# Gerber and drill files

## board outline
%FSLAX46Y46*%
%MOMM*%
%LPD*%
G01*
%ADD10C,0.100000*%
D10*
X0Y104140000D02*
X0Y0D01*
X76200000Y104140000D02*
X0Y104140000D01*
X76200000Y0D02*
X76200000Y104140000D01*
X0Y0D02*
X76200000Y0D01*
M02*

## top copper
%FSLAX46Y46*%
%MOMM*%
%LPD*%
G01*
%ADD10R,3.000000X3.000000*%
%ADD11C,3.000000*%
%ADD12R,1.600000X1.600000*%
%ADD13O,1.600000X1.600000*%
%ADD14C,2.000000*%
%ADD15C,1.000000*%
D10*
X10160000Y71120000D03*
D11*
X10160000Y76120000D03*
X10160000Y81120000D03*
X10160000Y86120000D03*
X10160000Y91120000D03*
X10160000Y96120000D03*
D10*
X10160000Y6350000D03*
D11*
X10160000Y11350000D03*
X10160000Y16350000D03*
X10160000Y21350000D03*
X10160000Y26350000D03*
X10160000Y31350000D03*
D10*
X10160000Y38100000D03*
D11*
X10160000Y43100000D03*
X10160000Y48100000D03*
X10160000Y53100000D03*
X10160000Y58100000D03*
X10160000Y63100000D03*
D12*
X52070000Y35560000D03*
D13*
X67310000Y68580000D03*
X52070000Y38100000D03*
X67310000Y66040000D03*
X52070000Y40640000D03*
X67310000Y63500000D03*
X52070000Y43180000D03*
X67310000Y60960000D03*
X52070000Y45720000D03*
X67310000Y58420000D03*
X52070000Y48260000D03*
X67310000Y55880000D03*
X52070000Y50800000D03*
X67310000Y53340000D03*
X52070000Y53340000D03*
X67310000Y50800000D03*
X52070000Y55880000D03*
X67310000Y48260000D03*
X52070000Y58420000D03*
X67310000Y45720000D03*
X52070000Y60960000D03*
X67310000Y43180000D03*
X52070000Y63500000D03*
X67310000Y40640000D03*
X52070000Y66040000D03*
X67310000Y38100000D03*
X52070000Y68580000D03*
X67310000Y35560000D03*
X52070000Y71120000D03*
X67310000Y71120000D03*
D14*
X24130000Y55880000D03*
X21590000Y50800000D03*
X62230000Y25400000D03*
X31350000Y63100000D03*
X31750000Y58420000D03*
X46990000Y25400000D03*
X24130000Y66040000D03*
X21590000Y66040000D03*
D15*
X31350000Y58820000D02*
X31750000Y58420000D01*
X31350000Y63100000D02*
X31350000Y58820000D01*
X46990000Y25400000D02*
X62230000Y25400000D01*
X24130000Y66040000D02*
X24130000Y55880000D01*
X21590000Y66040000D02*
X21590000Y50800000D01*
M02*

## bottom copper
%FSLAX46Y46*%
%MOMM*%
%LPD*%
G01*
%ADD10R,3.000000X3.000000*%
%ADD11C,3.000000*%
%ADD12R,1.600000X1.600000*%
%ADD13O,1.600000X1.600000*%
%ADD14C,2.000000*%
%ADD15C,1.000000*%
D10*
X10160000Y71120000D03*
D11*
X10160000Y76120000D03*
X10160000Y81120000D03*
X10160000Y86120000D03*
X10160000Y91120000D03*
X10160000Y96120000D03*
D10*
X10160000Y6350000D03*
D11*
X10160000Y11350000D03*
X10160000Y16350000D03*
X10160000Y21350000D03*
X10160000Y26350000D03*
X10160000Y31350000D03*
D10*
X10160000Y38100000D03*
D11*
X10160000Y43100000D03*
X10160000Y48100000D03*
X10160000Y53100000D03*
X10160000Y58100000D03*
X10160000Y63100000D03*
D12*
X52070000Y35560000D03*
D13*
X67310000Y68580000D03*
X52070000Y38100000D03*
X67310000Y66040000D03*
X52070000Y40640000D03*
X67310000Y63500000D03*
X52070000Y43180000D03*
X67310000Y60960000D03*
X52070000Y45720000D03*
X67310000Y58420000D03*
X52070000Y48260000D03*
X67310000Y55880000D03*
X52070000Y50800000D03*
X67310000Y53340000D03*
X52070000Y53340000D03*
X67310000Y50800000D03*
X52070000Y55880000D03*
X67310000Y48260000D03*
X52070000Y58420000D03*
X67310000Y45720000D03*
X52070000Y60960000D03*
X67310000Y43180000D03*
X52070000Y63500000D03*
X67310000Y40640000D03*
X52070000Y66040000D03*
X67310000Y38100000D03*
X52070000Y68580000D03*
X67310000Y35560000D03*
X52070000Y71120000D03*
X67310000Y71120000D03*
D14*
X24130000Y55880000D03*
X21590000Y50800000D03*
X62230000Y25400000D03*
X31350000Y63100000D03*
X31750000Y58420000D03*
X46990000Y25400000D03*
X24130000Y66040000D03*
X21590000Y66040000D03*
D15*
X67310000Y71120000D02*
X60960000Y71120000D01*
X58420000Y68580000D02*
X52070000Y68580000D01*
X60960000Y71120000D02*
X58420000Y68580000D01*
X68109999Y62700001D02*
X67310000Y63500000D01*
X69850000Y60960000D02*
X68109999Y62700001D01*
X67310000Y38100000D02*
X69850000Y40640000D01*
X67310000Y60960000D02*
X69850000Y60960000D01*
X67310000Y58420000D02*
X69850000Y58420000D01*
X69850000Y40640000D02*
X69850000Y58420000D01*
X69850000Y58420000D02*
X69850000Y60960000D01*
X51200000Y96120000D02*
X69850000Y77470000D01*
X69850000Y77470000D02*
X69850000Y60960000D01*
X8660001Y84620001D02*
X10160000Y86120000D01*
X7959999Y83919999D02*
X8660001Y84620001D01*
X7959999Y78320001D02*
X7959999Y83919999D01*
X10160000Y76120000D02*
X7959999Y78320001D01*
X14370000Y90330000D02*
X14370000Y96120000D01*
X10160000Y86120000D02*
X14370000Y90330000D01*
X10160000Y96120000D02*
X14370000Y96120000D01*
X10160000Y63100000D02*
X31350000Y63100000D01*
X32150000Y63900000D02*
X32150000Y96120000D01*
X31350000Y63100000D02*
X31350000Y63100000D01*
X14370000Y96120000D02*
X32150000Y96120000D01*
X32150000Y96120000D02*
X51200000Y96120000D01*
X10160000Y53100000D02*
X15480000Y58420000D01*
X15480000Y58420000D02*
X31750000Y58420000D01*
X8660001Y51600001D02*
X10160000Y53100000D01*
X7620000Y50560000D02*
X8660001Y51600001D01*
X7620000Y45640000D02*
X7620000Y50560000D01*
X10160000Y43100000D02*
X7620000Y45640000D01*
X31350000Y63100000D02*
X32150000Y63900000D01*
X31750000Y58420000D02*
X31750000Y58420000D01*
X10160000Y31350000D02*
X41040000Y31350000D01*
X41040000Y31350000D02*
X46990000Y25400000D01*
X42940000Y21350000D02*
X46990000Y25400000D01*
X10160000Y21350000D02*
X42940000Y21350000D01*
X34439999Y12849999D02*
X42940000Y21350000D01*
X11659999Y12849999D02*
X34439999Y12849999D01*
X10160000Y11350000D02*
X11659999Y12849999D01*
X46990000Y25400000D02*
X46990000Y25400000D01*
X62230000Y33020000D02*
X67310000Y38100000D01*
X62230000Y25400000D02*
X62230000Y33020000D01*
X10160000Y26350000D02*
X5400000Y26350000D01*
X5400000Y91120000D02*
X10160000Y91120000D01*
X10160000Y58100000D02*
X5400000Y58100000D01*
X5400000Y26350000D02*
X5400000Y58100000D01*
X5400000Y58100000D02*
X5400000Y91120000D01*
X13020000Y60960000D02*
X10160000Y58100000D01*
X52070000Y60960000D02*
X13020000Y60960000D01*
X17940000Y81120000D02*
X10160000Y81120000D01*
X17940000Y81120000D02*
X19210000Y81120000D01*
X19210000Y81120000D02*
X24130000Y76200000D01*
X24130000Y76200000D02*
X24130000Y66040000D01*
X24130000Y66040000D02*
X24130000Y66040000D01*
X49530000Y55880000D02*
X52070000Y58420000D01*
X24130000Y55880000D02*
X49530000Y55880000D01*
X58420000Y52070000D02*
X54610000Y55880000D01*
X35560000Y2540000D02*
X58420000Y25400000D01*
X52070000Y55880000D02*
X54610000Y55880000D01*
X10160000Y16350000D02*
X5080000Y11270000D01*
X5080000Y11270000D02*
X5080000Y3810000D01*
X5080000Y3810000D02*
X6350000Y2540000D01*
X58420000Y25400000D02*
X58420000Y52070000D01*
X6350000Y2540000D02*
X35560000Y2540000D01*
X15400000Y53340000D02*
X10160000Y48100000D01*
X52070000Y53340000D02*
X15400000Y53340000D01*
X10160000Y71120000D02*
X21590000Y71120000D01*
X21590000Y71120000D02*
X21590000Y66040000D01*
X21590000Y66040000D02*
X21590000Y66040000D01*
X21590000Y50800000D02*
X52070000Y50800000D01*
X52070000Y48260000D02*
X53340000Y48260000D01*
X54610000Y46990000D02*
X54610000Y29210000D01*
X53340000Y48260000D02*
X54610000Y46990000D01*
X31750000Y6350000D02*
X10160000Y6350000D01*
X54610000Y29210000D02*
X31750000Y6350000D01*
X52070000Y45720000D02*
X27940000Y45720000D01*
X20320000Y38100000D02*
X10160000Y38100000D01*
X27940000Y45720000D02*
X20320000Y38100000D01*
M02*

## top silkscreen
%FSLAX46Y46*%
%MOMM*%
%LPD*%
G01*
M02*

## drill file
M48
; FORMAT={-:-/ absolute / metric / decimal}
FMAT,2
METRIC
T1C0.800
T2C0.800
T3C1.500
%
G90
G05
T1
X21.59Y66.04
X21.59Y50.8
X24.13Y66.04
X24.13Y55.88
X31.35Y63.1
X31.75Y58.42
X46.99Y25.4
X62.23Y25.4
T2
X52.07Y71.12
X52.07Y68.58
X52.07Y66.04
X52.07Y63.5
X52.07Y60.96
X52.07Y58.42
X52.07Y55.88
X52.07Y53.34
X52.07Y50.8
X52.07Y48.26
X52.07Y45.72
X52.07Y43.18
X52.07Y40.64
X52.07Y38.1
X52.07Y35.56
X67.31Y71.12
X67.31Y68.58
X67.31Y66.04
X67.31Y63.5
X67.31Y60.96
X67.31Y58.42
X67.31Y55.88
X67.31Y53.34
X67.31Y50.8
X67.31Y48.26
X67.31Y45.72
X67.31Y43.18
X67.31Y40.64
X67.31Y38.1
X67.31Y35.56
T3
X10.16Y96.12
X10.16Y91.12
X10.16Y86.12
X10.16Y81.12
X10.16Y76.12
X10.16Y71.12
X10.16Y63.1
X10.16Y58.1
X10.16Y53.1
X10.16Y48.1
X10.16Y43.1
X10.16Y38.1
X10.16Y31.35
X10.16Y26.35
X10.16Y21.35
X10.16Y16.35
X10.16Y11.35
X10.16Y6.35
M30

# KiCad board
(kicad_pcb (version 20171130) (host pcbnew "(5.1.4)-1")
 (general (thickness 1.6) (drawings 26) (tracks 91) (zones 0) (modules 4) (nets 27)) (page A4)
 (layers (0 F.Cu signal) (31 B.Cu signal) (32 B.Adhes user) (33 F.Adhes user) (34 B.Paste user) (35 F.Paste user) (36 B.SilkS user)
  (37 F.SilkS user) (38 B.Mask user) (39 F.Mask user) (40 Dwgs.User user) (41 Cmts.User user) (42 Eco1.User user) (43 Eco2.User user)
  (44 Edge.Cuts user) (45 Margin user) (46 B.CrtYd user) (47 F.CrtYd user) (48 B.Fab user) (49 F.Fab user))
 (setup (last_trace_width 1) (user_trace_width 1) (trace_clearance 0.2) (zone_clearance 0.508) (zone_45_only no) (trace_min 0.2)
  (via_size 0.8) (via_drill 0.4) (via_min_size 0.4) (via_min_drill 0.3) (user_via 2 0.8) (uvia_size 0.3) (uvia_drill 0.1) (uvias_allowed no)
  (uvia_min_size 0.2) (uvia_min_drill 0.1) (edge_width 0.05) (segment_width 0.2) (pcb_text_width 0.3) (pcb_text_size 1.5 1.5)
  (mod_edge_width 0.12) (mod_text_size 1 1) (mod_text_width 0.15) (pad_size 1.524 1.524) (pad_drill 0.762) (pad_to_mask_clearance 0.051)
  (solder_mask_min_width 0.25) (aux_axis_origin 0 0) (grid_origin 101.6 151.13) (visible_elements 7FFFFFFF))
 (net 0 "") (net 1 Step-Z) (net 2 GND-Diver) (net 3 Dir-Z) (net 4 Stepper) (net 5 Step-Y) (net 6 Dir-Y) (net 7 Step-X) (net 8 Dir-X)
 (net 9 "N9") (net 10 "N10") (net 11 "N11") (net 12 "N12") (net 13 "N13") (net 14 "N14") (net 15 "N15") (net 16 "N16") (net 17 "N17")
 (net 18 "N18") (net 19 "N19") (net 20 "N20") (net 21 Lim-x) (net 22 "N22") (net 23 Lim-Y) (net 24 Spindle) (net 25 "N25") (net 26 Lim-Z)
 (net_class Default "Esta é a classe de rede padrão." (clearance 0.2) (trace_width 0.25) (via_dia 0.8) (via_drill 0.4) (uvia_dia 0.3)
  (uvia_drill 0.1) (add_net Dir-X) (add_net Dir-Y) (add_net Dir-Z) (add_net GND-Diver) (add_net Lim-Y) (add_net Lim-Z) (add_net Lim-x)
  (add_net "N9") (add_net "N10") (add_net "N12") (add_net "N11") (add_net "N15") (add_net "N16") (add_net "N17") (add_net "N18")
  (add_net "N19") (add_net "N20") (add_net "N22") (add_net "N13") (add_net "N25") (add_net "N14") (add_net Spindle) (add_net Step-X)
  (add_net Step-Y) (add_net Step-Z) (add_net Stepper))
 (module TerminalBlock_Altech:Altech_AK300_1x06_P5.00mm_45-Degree (layer B.Cu) (at 10.16 -71.12 90)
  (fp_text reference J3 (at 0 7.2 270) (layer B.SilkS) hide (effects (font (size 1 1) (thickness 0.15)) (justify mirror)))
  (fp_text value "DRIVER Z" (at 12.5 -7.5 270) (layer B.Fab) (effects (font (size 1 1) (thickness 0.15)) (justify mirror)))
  (pad 1 thru_hole rect (at 0 0 90) (size 3 3) (drill 1.5) (layers *.Cu *.Mask) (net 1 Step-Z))
  (pad 2 thru_hole circle (at 5 0 90) (size 3 3) (drill 1.5) (layers *.Cu *.Mask) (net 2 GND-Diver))
  (pad 3 thru_hole circle (at 10 0 90) (size 3 3) (drill 1.5) (layers *.Cu *.Mask) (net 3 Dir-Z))
  (pad 4 thru_hole circle (at 15 0 90) (size 3 3) (drill 1.5) (layers *.Cu *.Mask) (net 2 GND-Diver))
  (pad 5 thru_hole circle (at 20 0 90) (size 3 3) (drill 1.5) (layers *.Cu *.Mask) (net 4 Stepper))
  (pad 6 thru_hole circle (at 25 0 90) (size 3 3) (drill 1.5) (layers *.Cu *.Mask) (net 2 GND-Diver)))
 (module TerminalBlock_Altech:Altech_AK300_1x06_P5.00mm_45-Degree (layer B.Cu) (at 10.16 -6.35 90)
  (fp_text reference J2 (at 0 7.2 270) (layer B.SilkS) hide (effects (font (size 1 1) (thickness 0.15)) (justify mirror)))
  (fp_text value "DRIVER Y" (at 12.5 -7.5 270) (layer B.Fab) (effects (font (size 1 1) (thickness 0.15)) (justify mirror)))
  (pad 1 thru_hole rect (at 0 0 90) (size 3 3) (drill 1.5) (layers *.Cu *.Mask) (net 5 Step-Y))
  (pad 2 thru_hole circle (at 5 0 90) (size 3 3) (drill 1.5) (layers *.Cu *.Mask) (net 2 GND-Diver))
  (pad 3 thru_hole circle (at 10 0 90) (size 3 3) (drill 1.5) (layers *.Cu *.Mask) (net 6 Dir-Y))
  (pad 4 thru_hole circle (at 15 0 90) (size 3 3) (drill 1.5) (layers *.Cu *.Mask) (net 2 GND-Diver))
  (pad 5 thru_hole circle (at 20 0 90) (size 3 3) (drill 1.5) (layers *.Cu *.Mask) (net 4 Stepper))
  (pad 6 thru_hole circle (at 25 0 90) (size 3 3) (drill 1.5) (layers *.Cu *.Mask) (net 2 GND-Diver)))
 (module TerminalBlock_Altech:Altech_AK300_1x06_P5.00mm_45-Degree (layer B.Cu) (at 10.16 -38.1 90)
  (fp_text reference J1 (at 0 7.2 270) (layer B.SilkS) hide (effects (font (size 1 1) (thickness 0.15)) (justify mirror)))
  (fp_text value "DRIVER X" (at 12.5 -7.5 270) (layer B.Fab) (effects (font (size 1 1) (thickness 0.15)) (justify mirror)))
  (pad 1 thru_hole rect (at 0 0 90) (size 3 3) (drill 1.5) (layers *.Cu *.Mask) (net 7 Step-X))
  (pad 2 thru_hole circle (at 5 0 90) (size 3 3) (drill 1.5) (layers *.Cu *.Mask) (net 2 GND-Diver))
  (pad 3 thru_hole circle (at 10 0 90) (size 3 3) (drill 1.5) (layers *.Cu *.Mask) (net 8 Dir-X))
  (pad 4 thru_hole circle (at 15 0 90) (size 3 3) (drill 1.5) (layers *.Cu *.Mask) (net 2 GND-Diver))
  (pad 5 thru_hole circle (at 20 0 90) (size 3 3) (drill 1.5) (layers *.Cu *.Mask) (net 4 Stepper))
  (pad 6 thru_hole circle (at 25 0 90) (size 3 3) (drill 1.5) (layers *.Cu *.Mask) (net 2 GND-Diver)))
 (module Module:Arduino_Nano (layer B.Cu) (at 52.07 -35.56)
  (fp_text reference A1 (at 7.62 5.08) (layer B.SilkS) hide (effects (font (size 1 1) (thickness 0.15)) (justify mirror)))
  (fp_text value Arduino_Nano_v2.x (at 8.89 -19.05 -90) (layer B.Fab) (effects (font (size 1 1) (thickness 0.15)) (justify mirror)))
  (pad 1 thru_hole rect (at 0 0) (size 1.6 1.6) (drill 0.8) (layers *.Cu *.Mask) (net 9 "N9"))
  (pad 17 thru_hole oval (at 15.24 -33.02) (size 1.6 1.6) (drill 0.8) (layers *.Cu *.Mask) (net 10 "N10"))
  (pad 2 thru_hole oval (at 0 -2.54) (size 1.6 1.6) (drill 0.8) (layers *.Cu *.Mask) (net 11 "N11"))
  (pad 18 thru_hole oval (at 15.24 -30.48) (size 1.6 1.6) (drill 0.8) (layers *.Cu *.Mask) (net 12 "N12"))
  (pad 3 thru_hole oval (at 0 -5.08) (size 1.6 1.6) (drill 0.8) (layers *.Cu *.Mask) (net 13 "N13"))
  (pad 19 thru_hole oval (at 15.24 -27.94) (size 1.6 1.6) (drill 0.8) (layers *.Cu *.Mask) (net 2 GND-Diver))
  (pad 4 thru_hole oval (at 0 -7.62) (size 1.6 1.6) (drill 0.8) (layers *.Cu *.Mask) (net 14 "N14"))
  (pad 20 thru_hole oval (at 15.24 -25.4) (size 1.6 1.6) (drill 0.8) (layers *.Cu *.Mask) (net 2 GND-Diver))
  (pad 5 thru_hole oval (at 0 -10.16) (size 1.6 1.6) (drill 0.8) (layers *.Cu *.Mask) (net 7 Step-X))
  (pad 21 thru_hole oval (at 15.24 -22.86) (size 1.6 1.6) (drill 0.8) (layers *.Cu *.Mask) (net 2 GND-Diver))
  (pad 6 thru_hole oval (at 0 -12.7) (size 1.6 1.6) (drill 0.8) (layers *.Cu *.Mask) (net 5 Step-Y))
  (pad 22 thru_hole oval (at 15.24 -20.32) (size 1.6 1.6) (drill 0.8) (layers *.Cu *.Mask) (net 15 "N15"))
  (pad 7 thru_hole oval (at 0 -15.24) (size 1.6 1.6) (drill 0.8) (layers *.Cu *.Mask) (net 1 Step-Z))
  (pad 23 thru_hole oval (at 15.24 -17.78) (size 1.6 1.6) (drill 0.8) (layers *.Cu *.Mask) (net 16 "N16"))
  (pad 8 thru_hole oval (at 0 -17.78) (size 1.6 1.6) (drill 0.8) (layers *.Cu *.Mask) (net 8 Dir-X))
  (pad 24 thru_hole oval (at 15.24 -15.24) (size 1.6 1.6) (drill 0.8) (layers *.Cu *.Mask) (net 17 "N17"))
  (pad 9 thru_hole oval (at 0 -20.32) (size 1.6 1.6) (drill 0.8) (layers *.Cu *.Mask) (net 6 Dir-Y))
  (pad 25 thru_hole oval (at 15.24 -12.7) (size 1.6 1.6) (drill 0.8) (layers *.Cu *.Mask) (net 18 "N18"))
  (pad 10 thru_hole oval (at 0 -22.86) (size 1.6 1.6) (drill 0.8) (layers *.Cu *.Mask) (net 3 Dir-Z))
  (pad 26 thru_hole oval (at 15.24 -10.16) (size 1.6 1.6) (drill 0.8) (layers *.Cu *.Mask) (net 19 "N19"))
  (pad 11 thru_hole oval (at 0 -25.4) (size 1.6 1.6) (drill 0.8) (layers *.Cu *.Mask) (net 4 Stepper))
  (pad 27 thru_hole oval (at 15.24 -7.62) (size 1.6 1.6) (drill 0.8) (layers *.Cu *.Mask) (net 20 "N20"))
  (pad 12 thru_hole oval (at 0 -27.94) (size 1.6 1.6) (drill 0.8) (layers *.Cu *.Mask) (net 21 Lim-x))
  (pad 28 thru_hole oval (at 15.24 -5.08) (size 1.6 1.6) (drill 0.8) (layers *.Cu *.Mask) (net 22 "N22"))
  (pad 13 thru_hole oval (at 0 -30.48) (size 1.6 1.6) (drill 0.8) (layers *.Cu *.Mask) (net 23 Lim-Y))
  (pad 29 thru_hole oval (at 15.24 -2.54) (size 1.6 1.6) (drill 0.8) (layers *.Cu *.Mask) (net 2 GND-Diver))
  (pad 14 thru_hole oval (at 0 -33.02) (size 1.6 1.6) (drill 0.8) (layers *.Cu *.Mask) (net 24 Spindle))
  (pad 30 thru_hole oval (at 15.24 0) (size 1.6 1.6) (drill 0.8) (layers *.Cu *.Mask) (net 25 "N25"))
  (pad 15 thru_hole oval (at 0 -35.56) (size 1.6 1.6) (drill 0.8) (layers *.Cu *.Mask) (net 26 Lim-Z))
  (pad 16 thru_hole oval (at 15.24 -35.56) (size 1.6 1.6) (drill 0.8) (layers *.Cu *.Mask) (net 24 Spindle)))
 (gr_line (start 0 -104.14) (end 0 0) (layer Edge.Cuts) (width 0.1))
 (gr_line (start 76.2 -104.14) (end 0 -104.14) (layer Edge.Cuts) (width 0.1))
 (gr_line (start 76.2 0) (end 76.2 -104.14) (layer Edge.Cuts) (width 0.1))
 (gr_line (start 0 0) (end 76.2 0) (layer Edge.Cuts) (width 0.1))
 (via (at 24.13 -55.88) (size 2) (drill 0.8) (layers F.Cu B.Cu) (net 3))
 (via (at 21.59 -50.8) (size 2) (drill 0.8) (layers F.Cu B.Cu) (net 1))
 (via (at 62.23 -25.4) (size 2) (drill 0.8) (layers F.Cu B.Cu) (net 2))
 (segment (start 67.31 -71.12) (end 60.96 -71.12) (width 1) (layer B.Cu) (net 24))
 (segment (start 58.42 -68.58) (end 52.07 -68.58) (width 1) (layer B.Cu) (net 24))
 (segment (start 60.96 -71.12) (end 58.42 -68.58) (width 1) (layer B.Cu) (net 24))
 (segment (start 68.109999 -62.700001) (end 67.31 -63.5) (width 1) (layer B.Cu) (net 2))
 (segment (start 69.85 -60.96) (end 68.109999 -62.700001) (width 1) (layer B.Cu) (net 2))
 (segment (start 67.31 -38.1) (end 69.85 -40.64) (width 1) (layer B.Cu) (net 2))
 (segment (start 67.31 -60.96) (end 69.85 -60.96) (width 1) (layer B.Cu) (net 2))
 (segment (start 67.31 -58.42) (end 69.85 -58.42) (width 1) (layer B.Cu) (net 2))
 (segment (start 69.85 -40.64) (end 69.85 -58.42) (width 1) (layer B.Cu) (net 2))
 (segment (start 69.85 -58.42) (end 69.85 -60.96) (width 1) (layer B.Cu) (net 2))
 (segment (start 51.2 -96.12) (end 69.85 -77.47) (width 1) (layer B.Cu) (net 2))
 (segment (start 69.85 -77.47) (end 69.85 -60.96) (width 1) (layer B.Cu) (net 2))
 (segment (start 8.660001 -84.620001) (end 10.16 -86.12) (width 1) (layer B.Cu) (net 2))
 (segment (start 7.959999 -83.919999) (end 8.660001 -84.620001) (width 1) (layer B.Cu) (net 2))
 (segment (start 7.959999 -78.320001) (end 7.959999 -83.919999) (width 1) (layer B.Cu) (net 2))
 (segment (start 10.16 -76.12) (end 7.959999 -78.320001) (width 1) (layer B.Cu) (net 2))
 (segment (start 14.37 -90.33) (end 14.37 -96.12) (width 1) (layer B.Cu) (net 2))
 (segment (start 10.16 -86.12) (end 14.37 -90.33) (width 1) (layer B.Cu) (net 2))
 (segment (start 10.16 -96.12) (end 14.37 -96.12) (width 1) (layer B.Cu) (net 2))
 (segment (start 10.16 -63.1) (end 31.35 -63.1) (width 1) (layer B.Cu) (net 2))
 (segment (start 32.15 -63.9) (end 32.15 -96.12) (width 1) (layer B.Cu) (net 2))
 (segment (start 31.35 -63.1) (end 31.35 -63.1) (width 1) (layer B.Cu) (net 2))
 (segment (start 14.37 -96.12) (end 32.15 -96.12) (width 1) (layer B.Cu) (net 2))
 (segment (start 32.15 -96.12) (end 51.2 -96.12) (width 1) (layer B.Cu) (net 2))
 (segment (start 10.16 -53.1) (end 15.48 -58.42) (width 1) (layer B.Cu) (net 2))
 (segment (start 15.48 -58.42) (end 31.75 -58.42) (width 1) (layer B.Cu) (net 2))
 (segment (start 8.660001 -51.600001) (end 10.16 -53.1) (width 1) (layer B.Cu) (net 2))
 (segment (start 7.62 -50.56) (end 8.660001 -51.600001) (width 1) (layer B.Cu) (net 2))
 (segment (start 7.62 -45.64) (end 7.62 -50.56) (width 1) (layer B.Cu) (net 2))
 (segment (start 10.16 -43.1) (end 7.62 -45.64) (width 1) (layer B.Cu) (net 2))
 (segment (start 31.35 -63.1) (end 32.15 -63.9) (width 1) (layer B.Cu) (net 2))
 (via (at 31.35 -63.1) (size 2) (drill 0.8) (layers F.Cu B.Cu) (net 2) (status 1000000))
 (segment (start 31.75 -58.42) (end 31.75 -58.42) (width 1) (layer B.Cu) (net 2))
 (via (at 31.75 -58.42) (size 2) (drill 0.8) (layers F.Cu B.Cu) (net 2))
 (segment (start 10.16 -31.35) (end 41.04 -31.35) (width 1) (layer B.Cu) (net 2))
 (segment (start 41.04 -31.35) (end 46.99 -25.4) (width 1) (layer B.Cu) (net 2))
 (segment (start 42.94 -21.35) (end 46.99 -25.4) (width 1) (layer B.Cu) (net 2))
 (segment (start 10.16 -21.35) (end 42.94 -21.35) (width 1) (layer B.Cu) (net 2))
 (segment (start 34.439999 -12.849999) (end 42.94 -21.35) (width 1) (layer B.Cu) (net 2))
 (segment (start 11.659999 -12.849999) (end 34.439999 -12.849999) (width 1) (layer B.Cu) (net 2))
 (segment (start 10.16 -11.35) (end 11.659999 -12.849999) (width 1) (layer B.Cu) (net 2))
 (segment (start 46.99 -25.4) (end 46.99 -25.4) (width 1) (layer B.Cu) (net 2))
 (via (at 46.99 -25.4) (size 2) (drill 0.8) (layers F.Cu B.Cu) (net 2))
 (segment (start 62.23 -33.02) (end 67.31 -38.1) (width 1) (layer B.Cu) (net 2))
 (segment (start 62.23 -25.4) (end 62.23 -33.02) (width 1) (layer B.Cu) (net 2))
 (segment (start 31.35 -58.82) (end 31.75 -58.42) (width 1) (layer F.Cu) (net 2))
 (segment (start 31.35 -63.1) (end 31.35 -58.82) (width 1) (layer F.Cu) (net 2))
 (segment (start 46.99 -25.4) (end 62.23 -25.4) (width 1) (layer F.Cu) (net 2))
 (segment (start 10.16 -26.35) (end 5.4 -26.35) (width 1) (layer B.Cu) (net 4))
 (segment (start 5.4 -91.12) (end 10.16 -91.12) (width 1) (layer B.Cu) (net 4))
 (segment (start 10.16 -58.1) (end 5.4 -58.1) (width 1) (layer B.Cu) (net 4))
 (segment (start 5.4 -26.35) (end 5.4 -58.1) (width 1) (layer B.Cu) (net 4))
 (segment (start 5.4 -58.1) (end 5.4 -91.12) (width 1) (layer B.Cu) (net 4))
 (segment (start 13.02 -60.96) (end 10.16 -58.1) (width 1) (layer B.Cu) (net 4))
 (segment (start 52.07 -60.96) (end 13.02 -60.96) (width 1) (layer B.Cu) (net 4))
 (segment (start 17.94 -81.12) (end 10.16 -81.12) (width 1) (layer B.Cu) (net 3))
 (segment (start 17.94 -81.12) (end 19.21 -81.12) (width 1) (layer B.Cu) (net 3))
 (segment (start 19.21 -81.12) (end 24.13 -76.2) (width 1) (layer B.Cu) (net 3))
 (segment (start 24.13 -76.2) (end 24.13 -66.04) (width 1) (layer B.Cu) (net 3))
 (segment (start 24.13 -66.04) (end 24.13 -66.04) (width 1) (layer B.Cu) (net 3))
 (via (at 24.13 -66.04) (size 2) (drill 0.8) (layers F.Cu B.Cu) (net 3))
 (segment (start 49.53 -55.88) (end 52.07 -58.42) (width 1) (layer B.Cu) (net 3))
 (segment (start 24.13 -55.88) (end 49.53 -55.88) (width 1) (layer B.Cu) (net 3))
 (segment (start 24.13 -66.04) (end 24.13 -55.88) (width 1) (layer F.Cu) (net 3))
 (segment (start 58.42 -52.07) (end 54.61 -55.88) (width 1) (layer B.Cu) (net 6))
 (segment (start 35.56 -2.54) (end 58.42 -25.4) (width 1) (layer B.Cu) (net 6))
 (segment (start 52.07 -55.88) (end 54.61 -55.88) (width 1) (layer B.Cu) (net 6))
 (segment (start 10.16 -16.35) (end 5.08 -11.27) (width 1) (layer B.Cu) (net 6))
 (segment (start 5.08 -11.27) (end 5.08 -3.81) (width 1) (layer B.Cu) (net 6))
 (segment (start 5.08 -3.81) (end 6.35 -2.54) (width 1) (layer B.Cu) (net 6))
 (segment (start 58.42 -25.4) (end 58.42 -52.07) (width 1) (layer B.Cu) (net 6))
 (segment (start 6.35 -2.54) (end 35.56 -2.54) (width 1) (layer B.Cu) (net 6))
 (segment (start 15.4 -53.34) (end 10.16 -48.1) (width 1) (layer B.Cu) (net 8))
 (segment (start 52.07 -53.34) (end 15.4 -53.34) (width 1) (layer B.Cu) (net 8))
 (segment (start 10.16 -71.12) (end 21.59 -71.12) (width 1) (layer B.Cu) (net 1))
 (segment (start 21.59 -71.12) (end 21.59 -66.04) (width 1) (layer B.Cu) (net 1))
 (segment (start 21.59 -66.04) (end 21.59 -66.04) (width 1) (layer B.Cu) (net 1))
 (via (at 21.59 -66.04) (size 2) (drill 0.8) (layers F.Cu B.Cu) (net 1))
 (segment (start 21.59 -50.8) (end 52.07 -50.8) (width 1) (layer B.Cu) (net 1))
 (segment (start 21.59 -66.04) (end 21.59 -50.8) (width 1) (layer F.Cu) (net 1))
 (segment (start 52.07 -48.26) (end 53.34 -48.26) (width 1) (layer B.Cu) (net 5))
 (segment (start 54.61 -46.99) (end 54.61 -29.21) (width 1) (layer B.Cu) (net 5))
 (segment (start 53.34 -48.26) (end 54.61 -46.99) (width 1) (layer B.Cu) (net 5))
 (segment (start 31.75 -6.35) (end 10.16 -6.35) (width 1) (layer B.Cu) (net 5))
 (segment (start 54.61 -29.21) (end 31.75 -6.35) (width 1) (layer B.Cu) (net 5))
 (segment (start 52.07 -45.72) (end 27.94 -45.72) (width 1) (layer B.Cu) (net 7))
 (segment (start 20.32 -38.1) (end 10.16 -38.1) (width 1) (layer B.Cu) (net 7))
 (segment (start 27.94 -45.72) (end 20.32 -38.1) (width 1) (layer B.Cu) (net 7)))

